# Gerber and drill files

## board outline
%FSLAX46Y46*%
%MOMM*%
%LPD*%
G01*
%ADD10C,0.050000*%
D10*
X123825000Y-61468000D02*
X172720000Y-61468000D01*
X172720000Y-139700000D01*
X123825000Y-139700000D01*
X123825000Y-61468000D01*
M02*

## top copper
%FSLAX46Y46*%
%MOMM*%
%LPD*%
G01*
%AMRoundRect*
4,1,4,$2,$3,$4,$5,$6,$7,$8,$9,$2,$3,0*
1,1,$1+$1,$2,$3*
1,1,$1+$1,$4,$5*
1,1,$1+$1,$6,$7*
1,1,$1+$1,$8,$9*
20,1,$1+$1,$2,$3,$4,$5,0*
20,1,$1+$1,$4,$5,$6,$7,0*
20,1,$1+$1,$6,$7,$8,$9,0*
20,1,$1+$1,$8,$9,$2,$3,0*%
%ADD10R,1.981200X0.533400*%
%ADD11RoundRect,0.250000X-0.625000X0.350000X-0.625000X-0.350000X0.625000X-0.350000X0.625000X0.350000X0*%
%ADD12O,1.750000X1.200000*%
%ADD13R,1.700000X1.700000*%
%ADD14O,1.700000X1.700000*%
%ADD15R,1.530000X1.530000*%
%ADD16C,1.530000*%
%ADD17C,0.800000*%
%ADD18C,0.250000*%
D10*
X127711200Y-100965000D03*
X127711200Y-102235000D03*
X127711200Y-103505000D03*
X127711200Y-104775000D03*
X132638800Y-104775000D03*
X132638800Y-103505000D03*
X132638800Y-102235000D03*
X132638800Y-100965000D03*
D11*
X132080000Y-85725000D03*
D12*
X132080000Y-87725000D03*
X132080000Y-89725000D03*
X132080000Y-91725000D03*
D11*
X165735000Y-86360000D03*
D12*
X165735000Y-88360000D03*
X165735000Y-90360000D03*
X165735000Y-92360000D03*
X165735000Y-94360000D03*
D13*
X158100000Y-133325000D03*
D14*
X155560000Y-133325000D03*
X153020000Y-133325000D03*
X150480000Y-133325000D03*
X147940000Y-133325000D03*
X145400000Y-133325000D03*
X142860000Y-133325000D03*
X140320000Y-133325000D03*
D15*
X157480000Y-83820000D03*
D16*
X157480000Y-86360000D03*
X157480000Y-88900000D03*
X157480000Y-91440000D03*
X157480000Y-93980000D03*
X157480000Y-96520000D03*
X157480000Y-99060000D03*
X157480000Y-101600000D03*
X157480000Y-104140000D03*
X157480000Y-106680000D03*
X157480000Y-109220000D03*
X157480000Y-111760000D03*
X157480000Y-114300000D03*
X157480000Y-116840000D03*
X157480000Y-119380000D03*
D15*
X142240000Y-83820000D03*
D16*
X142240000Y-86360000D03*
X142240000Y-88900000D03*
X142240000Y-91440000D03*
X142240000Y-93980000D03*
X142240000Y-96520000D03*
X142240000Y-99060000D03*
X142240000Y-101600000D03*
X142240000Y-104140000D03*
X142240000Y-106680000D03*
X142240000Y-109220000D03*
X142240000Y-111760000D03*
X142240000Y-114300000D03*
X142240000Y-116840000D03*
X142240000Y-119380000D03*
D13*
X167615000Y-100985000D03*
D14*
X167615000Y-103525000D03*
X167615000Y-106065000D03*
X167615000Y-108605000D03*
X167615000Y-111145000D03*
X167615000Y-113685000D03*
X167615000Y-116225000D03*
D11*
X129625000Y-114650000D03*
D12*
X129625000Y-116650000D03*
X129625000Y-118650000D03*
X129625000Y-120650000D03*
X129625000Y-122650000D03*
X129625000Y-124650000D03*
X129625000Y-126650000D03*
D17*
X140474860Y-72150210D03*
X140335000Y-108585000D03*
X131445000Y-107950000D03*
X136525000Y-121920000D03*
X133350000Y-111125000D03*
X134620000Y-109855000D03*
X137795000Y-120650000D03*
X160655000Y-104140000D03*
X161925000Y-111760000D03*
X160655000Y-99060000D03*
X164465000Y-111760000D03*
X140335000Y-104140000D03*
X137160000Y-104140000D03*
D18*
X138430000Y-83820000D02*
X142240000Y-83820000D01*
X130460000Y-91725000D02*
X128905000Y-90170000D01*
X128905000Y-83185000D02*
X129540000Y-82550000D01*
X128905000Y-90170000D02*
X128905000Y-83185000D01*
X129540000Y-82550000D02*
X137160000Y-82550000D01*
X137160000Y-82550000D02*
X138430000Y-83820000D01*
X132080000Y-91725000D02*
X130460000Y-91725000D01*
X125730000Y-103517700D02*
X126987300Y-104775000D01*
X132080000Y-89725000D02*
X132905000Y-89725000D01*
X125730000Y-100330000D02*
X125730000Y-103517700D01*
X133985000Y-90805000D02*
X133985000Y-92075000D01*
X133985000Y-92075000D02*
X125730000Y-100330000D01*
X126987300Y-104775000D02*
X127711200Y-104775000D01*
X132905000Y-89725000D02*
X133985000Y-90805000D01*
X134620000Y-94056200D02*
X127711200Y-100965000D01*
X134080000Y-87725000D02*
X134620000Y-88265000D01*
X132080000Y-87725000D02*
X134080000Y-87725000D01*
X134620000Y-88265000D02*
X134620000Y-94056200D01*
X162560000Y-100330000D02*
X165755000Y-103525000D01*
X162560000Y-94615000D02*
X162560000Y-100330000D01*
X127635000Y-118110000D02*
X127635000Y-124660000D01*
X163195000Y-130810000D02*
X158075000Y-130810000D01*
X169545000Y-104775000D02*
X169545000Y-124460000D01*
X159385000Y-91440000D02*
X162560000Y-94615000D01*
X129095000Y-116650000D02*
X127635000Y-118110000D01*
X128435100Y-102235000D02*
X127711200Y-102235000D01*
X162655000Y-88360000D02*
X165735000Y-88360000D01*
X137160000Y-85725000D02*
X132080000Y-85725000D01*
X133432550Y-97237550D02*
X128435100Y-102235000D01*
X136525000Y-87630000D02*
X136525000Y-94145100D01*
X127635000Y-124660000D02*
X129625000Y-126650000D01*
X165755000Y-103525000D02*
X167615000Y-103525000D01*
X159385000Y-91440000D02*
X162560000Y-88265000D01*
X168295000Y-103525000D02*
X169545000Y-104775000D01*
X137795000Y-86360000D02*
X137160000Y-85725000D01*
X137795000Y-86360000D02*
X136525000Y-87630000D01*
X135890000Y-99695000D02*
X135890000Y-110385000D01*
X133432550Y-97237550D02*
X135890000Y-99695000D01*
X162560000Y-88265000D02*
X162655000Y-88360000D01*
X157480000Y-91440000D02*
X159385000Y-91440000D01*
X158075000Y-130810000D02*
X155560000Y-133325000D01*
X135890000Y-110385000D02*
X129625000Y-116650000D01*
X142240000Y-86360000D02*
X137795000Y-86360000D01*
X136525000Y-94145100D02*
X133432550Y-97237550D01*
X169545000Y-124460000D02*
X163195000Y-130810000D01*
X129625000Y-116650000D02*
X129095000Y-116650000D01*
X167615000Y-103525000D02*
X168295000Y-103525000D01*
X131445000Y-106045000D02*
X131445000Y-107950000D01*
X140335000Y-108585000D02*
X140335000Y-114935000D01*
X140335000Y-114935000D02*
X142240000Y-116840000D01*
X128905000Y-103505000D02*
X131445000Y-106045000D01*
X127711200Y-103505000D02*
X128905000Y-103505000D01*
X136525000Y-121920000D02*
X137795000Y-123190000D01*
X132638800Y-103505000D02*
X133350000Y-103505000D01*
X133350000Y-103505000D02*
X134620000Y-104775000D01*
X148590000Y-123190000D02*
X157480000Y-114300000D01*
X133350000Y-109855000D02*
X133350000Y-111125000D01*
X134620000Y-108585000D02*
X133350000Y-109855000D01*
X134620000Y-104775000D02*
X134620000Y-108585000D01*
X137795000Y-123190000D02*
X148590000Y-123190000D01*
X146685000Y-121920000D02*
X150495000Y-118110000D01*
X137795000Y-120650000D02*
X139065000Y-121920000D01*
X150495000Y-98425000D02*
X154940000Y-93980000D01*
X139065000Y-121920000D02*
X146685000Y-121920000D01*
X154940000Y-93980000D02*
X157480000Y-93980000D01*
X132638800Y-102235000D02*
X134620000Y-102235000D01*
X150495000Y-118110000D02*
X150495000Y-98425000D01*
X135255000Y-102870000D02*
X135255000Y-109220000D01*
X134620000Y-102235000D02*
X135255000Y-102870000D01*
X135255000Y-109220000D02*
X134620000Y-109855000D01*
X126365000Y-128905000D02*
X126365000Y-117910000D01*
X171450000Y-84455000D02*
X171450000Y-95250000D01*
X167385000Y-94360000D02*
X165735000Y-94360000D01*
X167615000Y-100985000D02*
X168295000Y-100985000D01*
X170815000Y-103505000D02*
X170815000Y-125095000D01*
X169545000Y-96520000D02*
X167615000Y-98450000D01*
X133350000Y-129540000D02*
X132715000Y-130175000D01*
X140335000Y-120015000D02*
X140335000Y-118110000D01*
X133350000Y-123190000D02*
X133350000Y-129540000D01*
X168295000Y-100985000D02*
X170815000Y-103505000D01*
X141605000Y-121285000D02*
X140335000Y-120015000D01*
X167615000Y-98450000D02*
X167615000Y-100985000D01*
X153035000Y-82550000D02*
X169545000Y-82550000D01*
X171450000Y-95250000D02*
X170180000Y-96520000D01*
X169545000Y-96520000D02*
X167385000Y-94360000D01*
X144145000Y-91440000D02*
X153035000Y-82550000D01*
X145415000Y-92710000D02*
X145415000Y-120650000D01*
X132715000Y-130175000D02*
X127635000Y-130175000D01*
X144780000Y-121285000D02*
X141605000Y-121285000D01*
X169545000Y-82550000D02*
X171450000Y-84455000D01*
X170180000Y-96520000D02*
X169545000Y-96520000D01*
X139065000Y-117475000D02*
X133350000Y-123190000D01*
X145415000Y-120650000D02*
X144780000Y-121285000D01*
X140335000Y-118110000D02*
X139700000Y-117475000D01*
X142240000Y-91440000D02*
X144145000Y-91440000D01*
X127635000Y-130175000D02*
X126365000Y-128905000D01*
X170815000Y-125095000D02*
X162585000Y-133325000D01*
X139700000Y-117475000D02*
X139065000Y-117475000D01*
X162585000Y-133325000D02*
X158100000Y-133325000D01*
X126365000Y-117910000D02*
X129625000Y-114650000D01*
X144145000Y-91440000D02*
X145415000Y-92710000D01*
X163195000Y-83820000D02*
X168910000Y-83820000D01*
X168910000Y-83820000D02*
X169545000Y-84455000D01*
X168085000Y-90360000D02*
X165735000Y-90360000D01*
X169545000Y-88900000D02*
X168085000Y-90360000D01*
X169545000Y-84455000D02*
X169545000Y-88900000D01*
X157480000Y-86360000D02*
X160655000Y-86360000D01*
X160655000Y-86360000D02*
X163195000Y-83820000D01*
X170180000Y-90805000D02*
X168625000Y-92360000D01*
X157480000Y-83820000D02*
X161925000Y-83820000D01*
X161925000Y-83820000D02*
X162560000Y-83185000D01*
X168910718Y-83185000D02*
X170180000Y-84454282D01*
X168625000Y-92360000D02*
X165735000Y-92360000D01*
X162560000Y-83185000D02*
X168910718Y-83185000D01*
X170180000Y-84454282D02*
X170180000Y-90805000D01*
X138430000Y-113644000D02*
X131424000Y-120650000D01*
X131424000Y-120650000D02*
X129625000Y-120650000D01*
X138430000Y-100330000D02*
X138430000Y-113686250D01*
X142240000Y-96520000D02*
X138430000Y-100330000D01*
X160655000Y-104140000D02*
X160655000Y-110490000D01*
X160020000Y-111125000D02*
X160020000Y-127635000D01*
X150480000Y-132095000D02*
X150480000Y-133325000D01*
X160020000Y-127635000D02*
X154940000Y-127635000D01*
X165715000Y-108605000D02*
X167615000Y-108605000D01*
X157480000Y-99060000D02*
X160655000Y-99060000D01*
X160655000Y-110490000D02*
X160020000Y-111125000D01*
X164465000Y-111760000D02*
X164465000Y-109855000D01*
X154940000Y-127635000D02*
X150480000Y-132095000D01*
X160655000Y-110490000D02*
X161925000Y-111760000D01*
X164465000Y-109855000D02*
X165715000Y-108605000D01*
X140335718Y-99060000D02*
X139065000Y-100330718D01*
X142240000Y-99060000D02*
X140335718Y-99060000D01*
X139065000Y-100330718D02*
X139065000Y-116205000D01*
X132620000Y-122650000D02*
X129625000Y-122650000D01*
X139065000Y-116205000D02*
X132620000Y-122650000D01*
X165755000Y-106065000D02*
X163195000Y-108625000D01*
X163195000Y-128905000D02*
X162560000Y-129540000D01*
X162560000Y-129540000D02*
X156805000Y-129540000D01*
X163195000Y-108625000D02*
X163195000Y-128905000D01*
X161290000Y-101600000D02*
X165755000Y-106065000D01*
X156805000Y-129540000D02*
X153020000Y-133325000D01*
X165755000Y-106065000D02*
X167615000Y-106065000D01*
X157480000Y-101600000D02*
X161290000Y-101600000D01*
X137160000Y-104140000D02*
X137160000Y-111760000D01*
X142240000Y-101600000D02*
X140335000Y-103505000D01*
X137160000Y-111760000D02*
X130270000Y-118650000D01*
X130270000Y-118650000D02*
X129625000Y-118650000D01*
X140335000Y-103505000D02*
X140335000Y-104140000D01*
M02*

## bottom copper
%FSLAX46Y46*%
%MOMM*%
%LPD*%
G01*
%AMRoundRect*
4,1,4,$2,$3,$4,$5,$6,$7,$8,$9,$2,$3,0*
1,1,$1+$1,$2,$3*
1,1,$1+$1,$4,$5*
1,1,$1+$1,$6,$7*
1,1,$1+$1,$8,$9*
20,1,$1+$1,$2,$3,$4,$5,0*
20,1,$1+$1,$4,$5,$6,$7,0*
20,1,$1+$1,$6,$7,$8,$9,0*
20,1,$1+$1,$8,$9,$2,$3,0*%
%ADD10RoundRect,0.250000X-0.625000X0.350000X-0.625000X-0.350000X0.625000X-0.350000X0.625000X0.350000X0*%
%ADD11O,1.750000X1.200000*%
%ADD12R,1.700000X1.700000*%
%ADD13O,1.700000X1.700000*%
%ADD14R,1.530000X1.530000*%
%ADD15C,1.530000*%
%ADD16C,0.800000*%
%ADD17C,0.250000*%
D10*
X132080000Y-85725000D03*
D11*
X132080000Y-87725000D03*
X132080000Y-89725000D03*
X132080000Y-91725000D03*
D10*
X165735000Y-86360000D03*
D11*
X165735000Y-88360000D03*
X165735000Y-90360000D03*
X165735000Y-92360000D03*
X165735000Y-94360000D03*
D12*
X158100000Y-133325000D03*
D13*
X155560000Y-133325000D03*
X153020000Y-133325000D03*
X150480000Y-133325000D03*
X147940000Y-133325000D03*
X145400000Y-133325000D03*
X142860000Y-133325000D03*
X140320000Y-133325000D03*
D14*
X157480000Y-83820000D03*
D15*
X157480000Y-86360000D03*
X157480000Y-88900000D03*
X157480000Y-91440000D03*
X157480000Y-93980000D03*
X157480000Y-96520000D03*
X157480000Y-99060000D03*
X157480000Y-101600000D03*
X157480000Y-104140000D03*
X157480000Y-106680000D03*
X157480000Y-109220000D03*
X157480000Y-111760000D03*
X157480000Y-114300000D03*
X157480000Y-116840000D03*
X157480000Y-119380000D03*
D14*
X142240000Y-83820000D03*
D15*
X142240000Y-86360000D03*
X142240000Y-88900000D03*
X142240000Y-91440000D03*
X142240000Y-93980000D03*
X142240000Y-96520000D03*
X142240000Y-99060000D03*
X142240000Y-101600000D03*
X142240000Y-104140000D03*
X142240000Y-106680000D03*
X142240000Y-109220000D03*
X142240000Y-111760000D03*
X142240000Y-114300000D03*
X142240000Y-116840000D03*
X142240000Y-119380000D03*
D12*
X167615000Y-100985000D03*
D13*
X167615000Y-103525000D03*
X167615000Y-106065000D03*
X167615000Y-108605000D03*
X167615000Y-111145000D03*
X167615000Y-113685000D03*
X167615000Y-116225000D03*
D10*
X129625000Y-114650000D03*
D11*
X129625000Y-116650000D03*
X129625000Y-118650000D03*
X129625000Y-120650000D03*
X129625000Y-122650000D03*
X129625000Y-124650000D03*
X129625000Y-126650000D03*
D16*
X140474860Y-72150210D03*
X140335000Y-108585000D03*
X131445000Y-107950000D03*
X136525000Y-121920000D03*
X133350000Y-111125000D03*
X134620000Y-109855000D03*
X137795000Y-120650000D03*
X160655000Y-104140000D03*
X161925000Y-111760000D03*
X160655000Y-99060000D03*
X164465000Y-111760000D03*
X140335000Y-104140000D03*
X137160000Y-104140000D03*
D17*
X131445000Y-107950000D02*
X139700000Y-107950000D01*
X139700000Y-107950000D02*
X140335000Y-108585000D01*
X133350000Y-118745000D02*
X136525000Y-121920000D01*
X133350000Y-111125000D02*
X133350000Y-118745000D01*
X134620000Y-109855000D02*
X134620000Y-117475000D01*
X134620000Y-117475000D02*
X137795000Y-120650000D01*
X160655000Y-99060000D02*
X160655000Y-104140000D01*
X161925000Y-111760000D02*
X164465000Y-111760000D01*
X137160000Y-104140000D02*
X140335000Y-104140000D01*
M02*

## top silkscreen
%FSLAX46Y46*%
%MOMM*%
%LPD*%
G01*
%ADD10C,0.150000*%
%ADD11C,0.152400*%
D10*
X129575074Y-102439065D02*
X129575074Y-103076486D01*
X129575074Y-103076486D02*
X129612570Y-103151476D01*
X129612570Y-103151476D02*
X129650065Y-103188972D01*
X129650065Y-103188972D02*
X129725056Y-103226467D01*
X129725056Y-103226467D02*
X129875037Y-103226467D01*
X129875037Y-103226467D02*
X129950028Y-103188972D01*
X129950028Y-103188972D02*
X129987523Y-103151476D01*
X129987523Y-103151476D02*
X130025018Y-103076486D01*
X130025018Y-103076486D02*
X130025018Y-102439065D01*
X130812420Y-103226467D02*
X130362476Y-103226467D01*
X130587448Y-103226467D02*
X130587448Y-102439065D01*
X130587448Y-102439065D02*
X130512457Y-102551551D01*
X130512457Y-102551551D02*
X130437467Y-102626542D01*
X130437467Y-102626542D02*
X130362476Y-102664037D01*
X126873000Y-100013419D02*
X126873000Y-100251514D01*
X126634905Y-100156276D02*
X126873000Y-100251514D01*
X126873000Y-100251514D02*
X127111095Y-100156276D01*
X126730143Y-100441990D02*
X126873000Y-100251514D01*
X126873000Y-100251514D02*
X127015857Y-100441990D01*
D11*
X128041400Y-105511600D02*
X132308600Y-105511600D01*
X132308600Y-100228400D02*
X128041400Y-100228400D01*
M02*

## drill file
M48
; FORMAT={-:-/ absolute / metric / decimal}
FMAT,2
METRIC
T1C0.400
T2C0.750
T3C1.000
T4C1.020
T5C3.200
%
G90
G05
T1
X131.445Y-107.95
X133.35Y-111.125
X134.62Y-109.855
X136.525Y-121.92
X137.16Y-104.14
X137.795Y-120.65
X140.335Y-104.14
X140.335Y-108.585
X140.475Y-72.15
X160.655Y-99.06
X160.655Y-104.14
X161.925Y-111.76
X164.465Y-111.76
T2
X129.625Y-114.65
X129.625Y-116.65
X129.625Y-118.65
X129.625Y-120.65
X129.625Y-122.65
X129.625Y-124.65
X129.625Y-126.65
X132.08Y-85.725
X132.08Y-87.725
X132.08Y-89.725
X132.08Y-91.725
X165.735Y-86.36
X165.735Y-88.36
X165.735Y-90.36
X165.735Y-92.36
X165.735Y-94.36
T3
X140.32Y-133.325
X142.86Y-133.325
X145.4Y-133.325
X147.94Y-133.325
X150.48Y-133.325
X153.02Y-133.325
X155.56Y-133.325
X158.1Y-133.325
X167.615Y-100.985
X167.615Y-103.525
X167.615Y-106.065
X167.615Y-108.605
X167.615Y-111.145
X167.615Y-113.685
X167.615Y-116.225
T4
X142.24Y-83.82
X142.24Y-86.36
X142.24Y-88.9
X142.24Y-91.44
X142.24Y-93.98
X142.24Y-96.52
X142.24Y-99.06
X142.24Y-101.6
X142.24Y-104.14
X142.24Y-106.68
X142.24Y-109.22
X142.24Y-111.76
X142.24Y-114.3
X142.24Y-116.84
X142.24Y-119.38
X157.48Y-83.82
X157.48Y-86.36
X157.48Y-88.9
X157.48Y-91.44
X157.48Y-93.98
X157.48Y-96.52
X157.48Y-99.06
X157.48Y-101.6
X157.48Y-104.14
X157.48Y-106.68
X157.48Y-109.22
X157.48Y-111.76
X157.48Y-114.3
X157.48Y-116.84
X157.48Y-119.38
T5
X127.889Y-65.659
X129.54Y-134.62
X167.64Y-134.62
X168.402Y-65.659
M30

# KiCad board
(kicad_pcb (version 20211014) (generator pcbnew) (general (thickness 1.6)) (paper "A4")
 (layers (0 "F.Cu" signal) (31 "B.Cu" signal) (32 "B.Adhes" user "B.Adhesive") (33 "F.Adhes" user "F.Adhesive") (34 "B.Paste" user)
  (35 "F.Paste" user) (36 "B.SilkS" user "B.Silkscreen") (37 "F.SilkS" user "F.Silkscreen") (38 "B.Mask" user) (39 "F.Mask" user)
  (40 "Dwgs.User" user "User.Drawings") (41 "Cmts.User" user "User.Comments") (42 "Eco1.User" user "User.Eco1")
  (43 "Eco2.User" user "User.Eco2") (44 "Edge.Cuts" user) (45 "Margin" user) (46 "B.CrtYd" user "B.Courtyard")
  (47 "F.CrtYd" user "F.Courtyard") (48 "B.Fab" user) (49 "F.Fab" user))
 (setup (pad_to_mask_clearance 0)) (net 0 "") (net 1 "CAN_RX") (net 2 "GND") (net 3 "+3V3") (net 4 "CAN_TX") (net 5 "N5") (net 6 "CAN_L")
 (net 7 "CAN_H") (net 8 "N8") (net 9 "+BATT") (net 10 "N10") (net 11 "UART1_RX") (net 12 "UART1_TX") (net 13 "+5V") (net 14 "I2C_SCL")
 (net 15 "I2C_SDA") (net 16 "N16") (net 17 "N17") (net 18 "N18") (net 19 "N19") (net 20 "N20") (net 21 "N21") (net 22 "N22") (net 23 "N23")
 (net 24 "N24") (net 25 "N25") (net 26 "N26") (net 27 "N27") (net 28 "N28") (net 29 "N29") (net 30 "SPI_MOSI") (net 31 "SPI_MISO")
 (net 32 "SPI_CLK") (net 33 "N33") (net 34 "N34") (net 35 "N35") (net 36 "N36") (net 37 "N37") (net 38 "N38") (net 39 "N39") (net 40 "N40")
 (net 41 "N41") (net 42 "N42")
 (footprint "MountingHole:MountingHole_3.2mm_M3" (layer "F.Cu") (at 168.402 65.659)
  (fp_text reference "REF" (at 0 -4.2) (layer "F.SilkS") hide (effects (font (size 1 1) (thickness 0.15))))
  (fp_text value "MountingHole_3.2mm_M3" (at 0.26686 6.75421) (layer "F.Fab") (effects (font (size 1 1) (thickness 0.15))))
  (pad "" np_thru_hole circle locked (at 0 0) (size 3.2 3.2) (drill 3.2) (layers *.Cu *.Mask)))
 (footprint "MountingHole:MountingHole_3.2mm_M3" (layer "F.Cu") (at 129.54 134.62)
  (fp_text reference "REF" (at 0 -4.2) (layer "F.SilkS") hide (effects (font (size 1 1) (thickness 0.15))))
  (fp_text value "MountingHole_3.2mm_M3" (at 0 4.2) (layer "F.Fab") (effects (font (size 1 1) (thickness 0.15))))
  (pad "" np_thru_hole circle locked (at 0 0) (size 3.2 3.2) (drill 3.2) (layers *.Cu *.Mask)))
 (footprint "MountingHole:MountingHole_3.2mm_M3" (layer "F.Cu") (at 167.64 134.62)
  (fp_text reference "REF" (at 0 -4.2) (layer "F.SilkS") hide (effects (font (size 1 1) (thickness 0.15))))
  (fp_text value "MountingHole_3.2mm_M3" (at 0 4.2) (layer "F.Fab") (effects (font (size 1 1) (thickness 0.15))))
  (pad "" np_thru_hole circle locked (at 0 0) (size 3.2 3.2) (drill 3.2) (layers *.Cu *.Mask)))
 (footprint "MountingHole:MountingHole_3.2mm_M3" (layer "F.Cu") (at 127.889 65.659)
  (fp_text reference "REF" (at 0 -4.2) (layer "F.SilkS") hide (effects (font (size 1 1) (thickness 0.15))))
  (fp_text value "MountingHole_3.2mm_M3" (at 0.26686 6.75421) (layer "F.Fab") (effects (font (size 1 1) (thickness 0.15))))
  (pad "" np_thru_hole circle locked (at 0 0) (size 3.2 3.2) (drill 3.2) (layers *.Cu *.Mask)))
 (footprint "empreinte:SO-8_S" (layer "F.Cu") (at 130.175 102.87)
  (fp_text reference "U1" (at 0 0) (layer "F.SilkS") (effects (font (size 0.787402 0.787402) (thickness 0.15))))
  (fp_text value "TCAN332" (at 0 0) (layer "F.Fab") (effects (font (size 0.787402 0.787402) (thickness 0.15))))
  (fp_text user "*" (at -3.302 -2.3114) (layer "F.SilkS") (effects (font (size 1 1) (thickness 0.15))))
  (fp_line (start -2.1336 2.6416) (end 2.1336 2.6416) (layer "F.SilkS") (width 0.1524))
  (fp_line (start 2.1336 -2.6416) (end -2.1336 -2.6416) (layer "F.SilkS") (width 0.1524))
  (pad "1" smd rect locked (at -2.4638 -1.905) (size 1.9812 0.5334) (layers "F.Cu" "F.Paste" "F.Mask") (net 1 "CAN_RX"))
  (pad "2" smd rect locked (at -2.4638 -0.635) (size 1.9812 0.5334) (layers "F.Cu" "F.Paste" "F.Mask") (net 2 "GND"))
  (pad "3" smd rect locked (at -2.4638 0.635) (size 1.9812 0.5334) (layers "F.Cu" "F.Paste" "F.Mask") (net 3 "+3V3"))
  (pad "4" smd rect locked (at -2.4638 1.905) (size 1.9812 0.5334) (layers "F.Cu" "F.Paste" "F.Mask") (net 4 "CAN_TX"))
  (pad "5" smd rect locked (at 2.4638 1.905) (size 1.9812 0.5334) (layers "F.Cu" "F.Paste" "F.Mask") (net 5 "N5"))
  (pad "6" smd rect locked (at 2.4638 0.635) (size 1.9812 0.5334) (layers "F.Cu" "F.Paste" "F.Mask") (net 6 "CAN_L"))
  (pad "7" smd rect locked (at 2.4638 -0.635) (size 1.9812 0.5334) (layers "F.Cu" "F.Paste" "F.Mask") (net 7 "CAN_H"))
  (pad "8" smd rect locked (at 2.4638 -1.905) (size 1.9812 0.5334) (layers "F.Cu" "F.Paste" "F.Mask") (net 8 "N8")))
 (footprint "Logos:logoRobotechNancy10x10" (layer "B.Cu") (at 160.15986 70.37221 180)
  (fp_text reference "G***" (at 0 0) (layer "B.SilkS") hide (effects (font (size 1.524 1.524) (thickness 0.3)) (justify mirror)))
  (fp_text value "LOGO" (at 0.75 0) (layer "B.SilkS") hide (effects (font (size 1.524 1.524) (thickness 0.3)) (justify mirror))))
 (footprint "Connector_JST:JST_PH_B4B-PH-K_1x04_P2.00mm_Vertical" (layer "B.Cu") (at 132.08 85.725 -90)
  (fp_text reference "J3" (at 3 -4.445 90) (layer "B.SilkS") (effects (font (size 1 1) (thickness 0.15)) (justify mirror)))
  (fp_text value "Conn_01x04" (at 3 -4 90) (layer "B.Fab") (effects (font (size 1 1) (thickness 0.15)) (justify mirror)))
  (pad "1" thru_hole roundrect locked (at 0 0 270) (size 1.2 1.75) (drill 0.75) (layers *.Cu *.Mask) (roundrect_rratio 0.208333)
   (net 2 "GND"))
  (pad "2" thru_hole oval locked (at 2 0 270) (size 1.2 1.75) (drill 0.75) (layers *.Cu *.Mask) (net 1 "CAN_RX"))
  (pad "3" thru_hole oval locked (at 4 0 270) (size 1.2 1.75) (drill 0.75) (layers *.Cu *.Mask) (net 4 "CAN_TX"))
  (pad "4" thru_hole oval locked (at 6 0 270) (size 1.2 1.75) (drill 0.75) (layers *.Cu *.Mask) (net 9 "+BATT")))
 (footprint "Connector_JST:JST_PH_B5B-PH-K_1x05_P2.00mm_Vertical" (layer "B.Cu") (at 165.735 86.36 -90)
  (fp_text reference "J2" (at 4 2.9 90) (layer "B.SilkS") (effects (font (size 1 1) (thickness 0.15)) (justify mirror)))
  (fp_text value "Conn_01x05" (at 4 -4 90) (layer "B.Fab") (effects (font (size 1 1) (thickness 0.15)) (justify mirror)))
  (pad "1" thru_hole roundrect locked (at 0 0 270) (size 1.2 1.75) (drill 0.75) (layers *.Cu *.Mask) (roundrect_rratio 0.208333)
   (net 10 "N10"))
  (pad "2" thru_hole oval locked (at 2 0 270) (size 1.2 1.75) (drill 0.75) (layers *.Cu *.Mask) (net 2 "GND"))
  (pad "3" thru_hole oval locked (at 4 0 270) (size 1.2 1.75) (drill 0.75) (layers *.Cu *.Mask) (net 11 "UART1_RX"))
  (pad "4" thru_hole oval locked (at 6 0 270) (size 1.2 1.75) (drill 0.75) (layers *.Cu *.Mask) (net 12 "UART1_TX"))
  (pad "5" thru_hole oval locked (at 8 0 270) (size 1.2 1.75) (drill 0.75) (layers *.Cu *.Mask) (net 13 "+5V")))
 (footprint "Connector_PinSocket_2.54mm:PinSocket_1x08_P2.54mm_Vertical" (layer "B.Cu") (at 158.1 133.325 90)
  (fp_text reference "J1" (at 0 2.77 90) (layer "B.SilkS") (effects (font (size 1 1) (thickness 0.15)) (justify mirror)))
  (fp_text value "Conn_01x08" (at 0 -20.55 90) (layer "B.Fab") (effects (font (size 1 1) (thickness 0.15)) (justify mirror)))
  (pad "1" thru_hole rect locked (at 0 0 90) (size 1.7 1.7) (drill 1) (layers *.Cu *.Mask) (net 13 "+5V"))
  (pad "2" thru_hole oval locked (at 0 -2.54 90) (size 1.7 1.7) (drill 1) (layers *.Cu *.Mask) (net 2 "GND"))
  (pad "3" thru_hole oval locked (at 0 -5.08 90) (size 1.7 1.7) (drill 1) (layers *.Cu *.Mask) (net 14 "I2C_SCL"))
  (pad "4" thru_hole oval locked (at 0 -7.62 90) (size 1.7 1.7) (drill 1) (layers *.Cu *.Mask) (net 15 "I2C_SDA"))
  (pad "5" thru_hole oval locked (at 0 -10.16 90) (size 1.7 1.7) (drill 1) (layers *.Cu *.Mask) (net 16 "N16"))
  (pad "6" thru_hole oval locked (at 0 -12.7 90) (size 1.7 1.7) (drill 1) (layers *.Cu *.Mask) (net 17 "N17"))
  (pad "7" thru_hole oval locked (at 0 -15.24 90) (size 1.7 1.7) (drill 1) (layers *.Cu *.Mask) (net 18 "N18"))
  (pad "8" thru_hole oval locked (at 0 -17.78 90) (size 1.7 1.7) (drill 1) (layers *.Cu *.Mask) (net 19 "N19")))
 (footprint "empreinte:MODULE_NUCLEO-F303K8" (layer "B.Cu") (at 149.86 101.6 180)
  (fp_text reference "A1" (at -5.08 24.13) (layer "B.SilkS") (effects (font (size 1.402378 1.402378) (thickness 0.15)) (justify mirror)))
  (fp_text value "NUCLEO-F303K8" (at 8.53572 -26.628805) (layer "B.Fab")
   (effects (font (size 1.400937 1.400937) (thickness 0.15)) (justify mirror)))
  (pad "3.1" thru_hole rect locked (at -7.62 17.78 180) (size 1.53 1.53) (drill 1.02) (layers *.Cu *.Mask) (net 12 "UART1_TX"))
  (pad "3.2" thru_hole circle locked (at -7.62 15.24 180) (size 1.53 1.53) (drill 1.02) (layers *.Cu *.Mask) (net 11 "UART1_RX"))
  (pad "3.3" thru_hole circle locked (at -7.62 12.7 180) (size 1.53 1.53) (drill 1.02) (layers *.Cu *.Mask) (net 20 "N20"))
  (pad "3.4" thru_hole circle locked (at -7.62 10.16 180) (size 1.53 1.53) (drill 1.02) (layers *.Cu *.Mask) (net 2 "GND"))
  (pad "3.5" thru_hole circle locked (at -7.62 7.62 180) (size 1.53 1.53) (drill 1.02) (layers *.Cu *.Mask) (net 7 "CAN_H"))
  (pad "3.6" thru_hole circle locked (at -7.62 5.08 180) (size 1.53 1.53) (drill 1.02) (layers *.Cu *.Mask) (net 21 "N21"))
  (pad "3.7" thru_hole circle locked (at -7.62 2.54 180) (size 1.53 1.53) (drill 1.02) (layers *.Cu *.Mask) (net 15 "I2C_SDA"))
  (pad "3.8" thru_hole circle locked (at -7.62 0 180) (size 1.53 1.53) (drill 1.02) (layers *.Cu *.Mask) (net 14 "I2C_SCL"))
  (pad "3.9" thru_hole circle locked (at -7.62 -2.54 180) (size 1.53 1.53) (drill 1.02) (layers *.Cu *.Mask) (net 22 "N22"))
  (pad "3.10" thru_hole circle locked (at -7.62 -5.08 180) (size 1.53 1.53) (drill 1.02) (layers *.Cu *.Mask) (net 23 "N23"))
  (pad "3.11" thru_hole circle locked (at -7.62 -7.62 180) (size 1.53 1.53) (drill 1.02) (layers *.Cu *.Mask) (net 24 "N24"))
  (pad "3.12" thru_hole circle locked (at -7.62 -10.16 180) (size 1.53 1.53) (drill 1.02) (layers *.Cu *.Mask) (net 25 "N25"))
  (pad "3.13" thru_hole circle locked (at -7.62 -12.7 180) (size 1.53 1.53) (drill 1.02) (layers *.Cu *.Mask) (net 6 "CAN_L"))
  (pad "3.14" thru_hole circle locked (at -7.62 -15.24 180) (size 1.53 1.53) (drill 1.02) (layers *.Cu *.Mask) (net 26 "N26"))
  (pad "3.15" thru_hole circle locked (at -7.62 -17.78 180) (size 1.53 1.53) (drill 1.02) (layers *.Cu *.Mask) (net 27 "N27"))
  (pad "4.1" thru_hole rect locked (at 7.62 17.78 180) (size 1.53 1.53) (drill 1.02) (layers *.Cu *.Mask) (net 9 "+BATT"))
  (pad "4.2" thru_hole circle locked (at 7.62 15.24 180) (size 1.53 1.53) (drill 1.02) (layers *.Cu *.Mask) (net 2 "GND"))
  (pad "4.3" thru_hole circle locked (at 7.62 12.7 180) (size 1.53 1.53) (drill 1.02) (layers *.Cu *.Mask) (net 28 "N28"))
  (pad "4.4" thru_hole circle locked (at 7.62 10.16 180) (size 1.53 1.53) (drill 1.02) (layers *.Cu *.Mask) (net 13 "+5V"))
  (pad "4.5" thru_hole circle locked (at 7.62 7.62 180) (size 1.53 1.53) (drill 1.02) (layers *.Cu *.Mask) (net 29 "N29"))
  (pad "4.6" thru_hole circle locked (at 7.62 5.08 180) (size 1.53 1.53) (drill 1.02) (layers *.Cu *.Mask) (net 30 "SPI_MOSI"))
  (pad "4.7" thru_hole circle locked (at 7.62 2.54 180) (size 1.53 1.53) (drill 1.02) (layers *.Cu *.Mask) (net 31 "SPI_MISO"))
  (pad "4.8" thru_hole circle locked (at 7.62 0 180) (size 1.53 1.53) (drill 1.02) (layers *.Cu *.Mask) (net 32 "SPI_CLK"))
  (pad "4.9" thru_hole circle locked (at 7.62 -2.54 180) (size 1.53 1.53) (drill 1.02) (layers *.Cu *.Mask) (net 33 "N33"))
  (pad "4.10" thru_hole circle locked (at 7.62 -5.08 180) (size 1.53 1.53) (drill 1.02) (layers *.Cu *.Mask) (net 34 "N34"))
  (pad "4.11" thru_hole circle locked (at 7.62 -7.62 180) (size 1.53 1.53) (drill 1.02) (layers *.Cu *.Mask) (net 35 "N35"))
  (pad "4.12" thru_hole circle locked (at 7.62 -10.16 180) (size 1.53 1.53) (drill 1.02) (layers *.Cu *.Mask) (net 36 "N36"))
  (pad "4.13" thru_hole circle locked (at 7.62 -12.7 180) (size 1.53 1.53) (drill 1.02) (layers *.Cu *.Mask) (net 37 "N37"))
  (pad "4.14" thru_hole circle locked (at 7.62 -15.24 180) (size 1.53 1.53) (drill 1.02) (layers *.Cu *.Mask) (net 3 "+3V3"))
  (pad "4.15" thru_hole circle locked (at 7.62 -17.78 180) (size 1.53 1.53) (drill 1.02) (layers *.Cu *.Mask) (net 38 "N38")))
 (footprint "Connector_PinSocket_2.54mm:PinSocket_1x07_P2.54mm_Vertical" (layer "B.Cu") (at 167.615 100.985 180)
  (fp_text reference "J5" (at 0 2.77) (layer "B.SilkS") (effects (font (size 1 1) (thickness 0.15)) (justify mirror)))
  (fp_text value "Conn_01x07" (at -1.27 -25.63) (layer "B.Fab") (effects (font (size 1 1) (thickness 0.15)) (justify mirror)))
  (pad "1" thru_hole rect locked (at 0 0 180) (size 1.7 1.7) (drill 1) (layers *.Cu *.Mask) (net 13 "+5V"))
  (pad "2" thru_hole oval locked (at 0 -2.54 180) (size 1.7 1.7) (drill 1) (layers *.Cu *.Mask) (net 2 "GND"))
  (pad "3" thru_hole oval locked (at 0 -5.08 180) (size 1.7 1.7) (drill 1) (layers *.Cu *.Mask) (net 14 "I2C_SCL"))
  (pad "4" thru_hole oval locked (at 0 -7.62 180) (size 1.7 1.7) (drill 1) (layers *.Cu *.Mask) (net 15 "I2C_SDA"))
  (pad "5" thru_hole oval locked (at 0 -10.16 180) (size 1.7 1.7) (drill 1) (layers *.Cu *.Mask) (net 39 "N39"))
  (pad "6" thru_hole oval locked (at 0 -12.7 180) (size 1.7 1.7) (drill 1) (layers *.Cu *.Mask) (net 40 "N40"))
  (pad "7" thru_hole oval locked (at 0 -15.24 180) (size 1.7 1.7) (drill 1) (layers *.Cu *.Mask) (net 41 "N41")))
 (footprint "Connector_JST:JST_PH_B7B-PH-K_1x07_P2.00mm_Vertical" (layer "B.Cu") (at 129.625 114.65 -90)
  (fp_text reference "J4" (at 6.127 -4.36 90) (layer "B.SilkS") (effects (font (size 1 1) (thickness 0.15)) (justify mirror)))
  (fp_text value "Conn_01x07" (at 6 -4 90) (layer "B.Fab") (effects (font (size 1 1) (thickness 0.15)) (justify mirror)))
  (pad "1" thru_hole roundrect locked (at 0 0 270) (size 1.2 1.75) (drill 0.75) (layers *.Cu *.Mask) (roundrect_rratio 0.208333)
   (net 13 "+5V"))
  (pad "2" thru_hole oval locked (at 2 0 270) (size 1.2 1.75) (drill 0.75) (layers *.Cu *.Mask) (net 2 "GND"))
  (pad "3" thru_hole oval locked (at 4 0 270) (size 1.2 1.75) (drill 0.75) (layers *.Cu *.Mask) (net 32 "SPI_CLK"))
  (pad "4" thru_hole oval locked (at 6 0 270) (size 1.2 1.75) (drill 0.75) (layers *.Cu *.Mask) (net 30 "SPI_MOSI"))
  (pad "5" thru_hole oval locked (at 8 0 270) (size 1.2 1.75) (drill 0.75) (layers *.Cu *.Mask) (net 31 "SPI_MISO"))
  (pad "6" thru_hole oval locked (at 10 0 270) (size 1.2 1.75) (drill 0.75) (layers *.Cu *.Mask) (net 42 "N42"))
  (pad "7" thru_hole oval locked (at 12 0 270) (size 1.2 1.75) (drill 0.75) (layers *.Cu *.Mask) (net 2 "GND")))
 (gr_rect (start 123.825 61.468) (end 172.72 139.7) (layer "Edge.Cuts") (width 0.05) (fill none))
 (via (at 140.47486 72.15021) (size 0.8) (drill 0.4) (layers "F.Cu" "B.Cu") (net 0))
 (segment (start 138.43 83.82) (end 142.24 83.82) (width 0.25) (layer "F.Cu") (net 9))
 (segment (start 130.46 91.725) (end 128.905 90.17) (width 0.25) (layer "F.Cu") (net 9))
 (segment (start 128.905 83.185) (end 129.54 82.55) (width 0.25) (layer "F.Cu") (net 9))
 (segment (start 128.905 90.17) (end 128.905 83.185) (width 0.25) (layer "F.Cu") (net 9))
 (segment (start 129.54 82.55) (end 137.16 82.55) (width 0.25) (layer "F.Cu") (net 9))
 (segment (start 137.16 82.55) (end 138.43 83.82) (width 0.25) (layer "F.Cu") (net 9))
 (segment (start 132.08 91.725) (end 130.46 91.725) (width 0.25) (layer "F.Cu") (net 9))
 (segment (start 125.73 103.5177) (end 126.9873 104.775) (width 0.25) (layer "F.Cu") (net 4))
 (segment (start 132.08 89.725) (end 132.905 89.725) (width 0.25) (layer "F.Cu") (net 4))
 (segment (start 125.73 100.33) (end 125.73 103.5177) (width 0.25) (layer "F.Cu") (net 4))
 (segment (start 133.985 90.805) (end 133.985 92.075) (width 0.25) (layer "F.Cu") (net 4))
 (segment (start 133.985 92.075) (end 125.73 100.33) (width 0.25) (layer "F.Cu") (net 4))
 (segment (start 126.9873 104.775) (end 127.7112 104.775) (width 0.25) (layer "F.Cu") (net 4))
 (segment (start 132.905 89.725) (end 133.985 90.805) (width 0.25) (layer "F.Cu") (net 4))
 (segment (start 134.62 94.0562) (end 127.7112 100.965) (width 0.25) (layer "F.Cu") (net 1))
 (segment (start 134.08 87.725) (end 134.62 88.265) (width 0.25) (layer "F.Cu") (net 1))
 (segment (start 132.08 87.725) (end 134.08 87.725) (width 0.25) (layer "F.Cu") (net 1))
 (segment (start 134.62 88.265) (end 134.62 94.0562) (width 0.25) (layer "F.Cu") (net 1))
 (segment (start 162.56 100.33) (end 165.755 103.525) (width 0.25) (layer "F.Cu") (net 2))
 (segment (start 162.56 94.615) (end 162.56 100.33) (width 0.25) (layer "F.Cu") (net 2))
 (segment (start 127.635 118.11) (end 127.635 124.66) (width 0.25) (layer "F.Cu") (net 2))
 (segment (start 163.195 130.81) (end 158.075 130.81) (width 0.25) (layer "F.Cu") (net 2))
 (segment (start 169.545 104.775) (end 169.545 124.46) (width 0.25) (layer "F.Cu") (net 2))
 (segment (start 159.385 91.44) (end 162.56 94.615) (width 0.25) (layer "F.Cu") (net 2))
 (segment (start 129.095 116.65) (end 127.635 118.11) (width 0.25) (layer "F.Cu") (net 2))
 (segment (start 128.4351 102.235) (end 127.7112 102.235) (width 0.25) (layer "F.Cu") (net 2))
 (segment (start 162.655 88.36) (end 165.735 88.36) (width 0.25) (layer "F.Cu") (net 2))
 (segment (start 137.16 85.725) (end 132.08 85.725) (width 0.25) (layer "F.Cu") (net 2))
 (segment (start 133.43255 97.23755) (end 128.4351 102.235) (width 0.25) (layer "F.Cu") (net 2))
 (segment (start 136.525 87.63) (end 136.525 94.1451) (width 0.25) (layer "F.Cu") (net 2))
 (segment (start 127.635 124.66) (end 129.625 126.65) (width 0.25) (layer "F.Cu") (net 2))
 (segment (start 165.755 103.525) (end 167.615 103.525) (width 0.25) (layer "F.Cu") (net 2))
 (segment (start 159.385 91.44) (end 162.56 88.265) (width 0.25) (layer "F.Cu") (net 2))
 (segment (start 168.295 103.525) (end 169.545 104.775) (width 0.25) (layer "F.Cu") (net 2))
 (segment (start 137.795 86.36) (end 137.16 85.725) (width 0.25) (layer "F.Cu") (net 2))
 (segment (start 137.795 86.36) (end 136.525 87.63) (width 0.25) (layer "F.Cu") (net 2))
 (segment (start 135.89 99.695) (end 135.89 110.385) (width 0.25) (layer "F.Cu") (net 2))
 (segment (start 133.43255 97.23755) (end 135.89 99.695) (width 0.25) (layer "F.Cu") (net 2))
 (segment (start 162.56 88.265) (end 162.655 88.36) (width 0.25) (layer "F.Cu") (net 2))
 (segment (start 157.48 91.44) (end 159.385 91.44) (width 0.25) (layer "F.Cu") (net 2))
 (segment (start 158.075 130.81) (end 155.56 133.325) (width 0.25) (layer "F.Cu") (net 2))
 (segment (start 135.89 110.385) (end 129.625 116.65) (width 0.25) (layer "F.Cu") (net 2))
 (segment (start 142.24 86.36) (end 137.795 86.36) (width 0.25) (layer "F.Cu") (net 2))
 (segment (start 136.525 94.1451) (end 133.43255 97.23755) (width 0.25) (layer "F.Cu") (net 2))
 (segment (start 169.545 124.46) (end 163.195 130.81) (width 0.25) (layer "F.Cu") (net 2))
 (segment (start 129.625 116.65) (end 129.095 116.65) (width 0.25) (layer "F.Cu") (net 2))
 (segment (start 167.615 103.525) (end 168.295 103.525) (width 0.25) (layer "F.Cu") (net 2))
 (segment (start 131.445 106.045) (end 131.445 107.95) (width 0.25) (layer "F.Cu") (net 3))
 (segment (start 140.335 108.585) (end 140.335 114.935) (width 0.25) (layer "F.Cu") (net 3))
 (segment (start 140.335 114.935) (end 142.24 116.84) (width 0.25) (layer "F.Cu") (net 3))
 (segment (start 128.905 103.505) (end 131.445 106.045) (width 0.25) (layer "F.Cu") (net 3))
 (segment (start 127.7112 103.505) (end 128.905 103.505) (width 0.25) (layer "F.Cu") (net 3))
 (via (at 140.335 108.585) (size 0.8) (drill 0.4) (layers "F.Cu" "B.Cu") (free) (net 3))
 (via (at 131.445 107.95) (size 0.8) (drill 0.4) (layers "F.Cu" "B.Cu") (free) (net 3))
 (segment (start 131.445 107.95) (end 139.7 107.95) (width 0.25) (layer "B.Cu") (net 3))
 (segment (start 139.7 107.95) (end 140.335 108.585) (width 0.25) (layer "B.Cu") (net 3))
 (segment (start 136.525 121.92) (end 137.795 123.19) (width 0.25) (layer "F.Cu") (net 6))
 (segment (start 132.6388 103.505) (end 133.35 103.505) (width 0.25) (layer "F.Cu") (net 6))
 (segment (start 133.35 103.505) (end 134.62 104.775) (width 0.25) (layer "F.Cu") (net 6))
 (segment (start 148.59 123.19) (end 157.48 114.3) (width 0.25) (layer "F.Cu") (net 6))
 (segment (start 133.35 109.855) (end 133.35 111.125) (width 0.25) (layer "F.Cu") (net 6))
 (segment (start 134.62 108.585) (end 133.35 109.855) (width 0.25) (layer "F.Cu") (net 6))
 (segment (start 134.62 104.775) (end 134.62 108.585) (width 0.25) (layer "F.Cu") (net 6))
 (segment (start 137.795 123.19) (end 148.59 123.19) (width 0.25) (layer "F.Cu") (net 6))
 (via (at 136.525 121.92) (size 0.8) (drill 0.4) (layers "F.Cu" "B.Cu") (free) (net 6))
 (via (at 133.35 111.125) (size 0.8) (drill 0.4) (layers "F.Cu" "B.Cu") (free) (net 6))
 (segment (start 133.35 118.745) (end 136.525 121.92) (width 0.25) (layer "B.Cu") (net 6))
 (segment (start 133.35 111.125) (end 133.35 118.745) (width 0.25) (layer "B.Cu") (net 6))
 (segment (start 146.685 121.92) (end 150.495 118.11) (width 0.25) (layer "F.Cu") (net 7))
 (segment (start 137.795 120.65) (end 139.065 121.92) (width 0.25) (layer "F.Cu") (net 7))
 (segment (start 150.495 98.425) (end 154.94 93.98) (width 0.25) (layer "F.Cu") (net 7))
 (segment (start 139.065 121.92) (end 146.685 121.92) (width 0.25) (layer "F.Cu") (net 7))
 (segment (start 154.94 93.98) (end 157.48 93.98) (width 0.25) (layer "F.Cu") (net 7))
 (segment (start 132.6388 102.235) (end 134.62 102.235) (width 0.25) (layer "F.Cu") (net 7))
 (segment (start 150.495 118.11) (end 150.495 98.425) (width 0.25) (layer "F.Cu") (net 7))
 (segment (start 135.255 102.87) (end 135.255 109.22) (width 0.25) (layer "F.Cu") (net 7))
 (segment (start 134.62 102.235) (end 135.255 102.87) (width 0.25) (layer "F.Cu") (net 7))
 (segment (start 135.255 109.22) (end 134.62 109.855) (width 0.25) (layer "F.Cu") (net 7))
 (via (at 134.62 109.855) (size 0.8) (drill 0.4) (layers "F.Cu" "B.Cu") (free) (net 7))
 (via (at 137.795 120.65) (size 0.8) (drill 0.4) (layers "F.Cu" "B.Cu") (free) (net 7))
 (segment (start 134.62 109.855) (end 134.62 117.475) (width 0.25) (layer "B.Cu") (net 7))
 (segment (start 134.62 117.475) (end 137.795 120.65) (width 0.25) (layer "B.Cu") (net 7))
 (segment (start 126.365 128.905) (end 126.365 117.91) (width 0.25) (layer "F.Cu") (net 13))
 (segment (start 171.45 84.455) (end 171.45 95.25) (width 0.25) (layer "F.Cu") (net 13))
 (segment (start 167.385 94.36) (end 165.735 94.36) (width 0.25) (layer "F.Cu") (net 13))
 (segment (start 167.615 100.985) (end 168.295 100.985) (width 0.25) (layer "F.Cu") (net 13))
 (segment (start 170.815 103.505) (end 170.815 125.095) (width 0.25) (layer "F.Cu") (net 13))
 (segment (start 169.545 96.52) (end 167.615 98.45) (width 0.25) (layer "F.Cu") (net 13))
 (segment (start 133.35 129.54) (end 132.715 130.175) (width 0.25) (layer "F.Cu") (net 13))
 (segment (start 140.335 120.015) (end 140.335 118.11) (width 0.25) (layer "F.Cu") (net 13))
 (segment (start 133.35 123.19) (end 133.35 129.54) (width 0.25) (layer "F.Cu") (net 13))
 (segment (start 168.295 100.985) (end 170.815 103.505) (width 0.25) (layer "F.Cu") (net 13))
 (segment (start 141.605 121.285) (end 140.335 120.015) (width 0.25) (layer "F.Cu") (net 13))
 (segment (start 167.615 98.45) (end 167.615 100.985) (width 0.25) (layer "F.Cu") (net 13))
 (segment (start 153.035 82.55) (end 169.545 82.55) (width 0.25) (layer "F.Cu") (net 13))
 (segment (start 171.45 95.25) (end 170.18 96.52) (width 0.25) (layer "F.Cu") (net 13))
 (segment (start 169.545 96.52) (end 167.385 94.36) (width 0.25) (layer "F.Cu") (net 13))
 (segment (start 144.145 91.44) (end 153.035 82.55) (width 0.25) (layer "F.Cu") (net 13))
 (segment (start 145.415 92.71) (end 145.415 120.65) (width 0.25) (layer "F.Cu") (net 13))
 (segment (start 132.715 130.175) (end 127.635 130.175) (width 0.25) (layer "F.Cu") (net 13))
 (segment (start 144.78 121.285) (end 141.605 121.285) (width 0.25) (layer "F.Cu") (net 13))
 (segment (start 169.545 82.55) (end 171.45 84.455) (width 0.25) (layer "F.Cu") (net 13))
 (segment (start 170.18 96.52) (end 169.545 96.52) (width 0.25) (layer "F.Cu") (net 13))
 (segment (start 139.065 117.475) (end 133.35 123.19) (width 0.25) (layer "F.Cu") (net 13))
 (segment (start 145.415 120.65) (end 144.78 121.285) (width 0.25) (layer "F.Cu") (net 13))
 (segment (start 140.335 118.11) (end 139.7 117.475) (width 0.25) (layer "F.Cu") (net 13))
 (segment (start 142.24 91.44) (end 144.145 91.44) (width 0.25) (layer "F.Cu") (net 13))
 (segment (start 127.635 130.175) (end 126.365 128.905) (width 0.25) (layer "F.Cu") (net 13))
 (segment (start 170.815 125.095) (end 162.585 133.325) (width 0.25) (layer "F.Cu") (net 13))
 (segment (start 139.7 117.475) (end 139.065 117.475) (width 0.25) (layer "F.Cu") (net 13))
 (segment (start 162.585 133.325) (end 158.1 133.325) (width 0.25) (layer "F.Cu") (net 13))
 (segment (start 126.365 117.91) (end 129.625 114.65) (width 0.25) (layer "F.Cu") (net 13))
 (segment (start 144.145 91.44) (end 145.415 92.71) (width 0.25) (layer "F.Cu") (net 13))
 (segment (start 163.195 83.82) (end 168.91 83.82) (width 0.25) (layer "F.Cu") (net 11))
 (segment (start 168.91 83.82) (end 169.545 84.455) (width 0.25) (layer "F.Cu") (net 11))
 (segment (start 168.085 90.36) (end 165.735 90.36) (width 0.25) (layer "F.Cu") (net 11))
 (segment (start 169.545 88.9) (end 168.085 90.36) (width 0.25) (layer "F.Cu") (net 11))
 (segment (start 169.545 84.455) (end 169.545 88.9) (width 0.25) (layer "F.Cu") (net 11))
 (segment (start 157.48 86.36) (end 160.655 86.36) (width 0.25) (layer "F.Cu") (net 11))
 (segment (start 160.655 86.36) (end 163.195 83.82) (width 0.25) (layer "F.Cu") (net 11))
 (segment (start 170.18 90.805) (end 168.625 92.36) (width 0.25) (layer "F.Cu") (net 12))
 (segment (start 157.48 83.82) (end 161.925 83.82) (width 0.25) (layer "F.Cu") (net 12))
 (segment (start 161.925 83.82) (end 162.56 83.185) (width 0.25) (layer "F.Cu") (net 12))
 (segment (start 168.910718 83.185) (end 170.18 84.454282) (width 0.25) (layer "F.Cu") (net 12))
 (segment (start 168.625 92.36) (end 165.735 92.36) (width 0.25) (layer "F.Cu") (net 12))
 (segment (start 162.56 83.185) (end 168.910718 83.185) (width 0.25) (layer "F.Cu") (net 12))
 (segment (start 170.18 84.454282) (end 170.18 90.805) (width 0.25) (layer "F.Cu") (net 12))
 (segment (start 138.43 113.644) (end 131.424 120.65) (width 0.25) (layer "F.Cu") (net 30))
 (segment (start 131.424 120.65) (end 129.625 120.65) (width 0.25) (layer "F.Cu") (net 30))
 (segment (start 138.43 100.33) (end 138.43 113.68625) (width 0.25) (layer "F.Cu") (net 30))
 (segment (start 142.24 96.52) (end 138.43 100.33) (width 0.25) (layer "F.Cu") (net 30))
 (segment (start 160.655 104.14) (end 160.655 110.49) (width 0.25) (layer "F.Cu") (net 15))
 (segment (start 160.02 111.125) (end 160.02 127.635) (width 0.25) (layer "F.Cu") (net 15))
 (segment (start 150.48 132.095) (end 150.48 133.325) (width 0.25) (layer "F.Cu") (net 15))
 (segment (start 160.02 127.635) (end 154.94 127.635) (width 0.25) (layer "F.Cu") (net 15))
 (segment (start 165.715 108.605) (end 167.615 108.605) (width 0.25) (layer "F.Cu") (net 15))
 (segment (start 157.48 99.06) (end 160.655 99.06) (width 0.25) (layer "F.Cu") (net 15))
 (segment (start 160.655 110.49) (end 160.02 111.125) (width 0.25) (layer "F.Cu") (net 15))
 (segment (start 164.465 111.76) (end 164.465 109.855) (width 0.25) (layer "F.Cu") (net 15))
 (segment (start 154.94 127.635) (end 150.48 132.095) (width 0.25) (layer "F.Cu") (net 15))
 (segment (start 160.655 110.49) (end 161.925 111.76) (width 0.25) (layer "F.Cu") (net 15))
 (segment (start 164.465 109.855) (end 165.715 108.605) (width 0.25) (layer "F.Cu") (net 15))
 (via (at 160.655 104.14) (size 0.8) (drill 0.4) (layers "F.Cu" "B.Cu") (free) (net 15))
 (via (at 161.925 111.76) (size 0.8) (drill 0.4) (layers "F.Cu" "B.Cu") (free) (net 15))
 (via (at 160.655 99.06) (size 0.8) (drill 0.4) (layers "F.Cu" "B.Cu") (free) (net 15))
 (via (at 164.465 111.76) (size 0.8) (drill 0.4) (layers "F.Cu" "B.Cu") (free) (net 15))
 (segment (start 160.655 99.06) (end 160.655 104.14) (width 0.25) (layer "B.Cu") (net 15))
 (segment (start 161.925 111.76) (end 164.465 111.76) (width 0.25) (layer "B.Cu") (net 15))
 (segment (start 140.335718 99.06) (end 139.065 100.330718) (width 0.25) (layer "F.Cu") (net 31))
 (segment (start 142.24 99.06) (end 140.335718 99.06) (width 0.25) (layer "F.Cu") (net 31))
 (segment (start 139.065 100.330718) (end 139.065 116.205) (width 0.25) (layer "F.Cu") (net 31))
 (segment (start 132.62 122.65) (end 129.625 122.65) (width 0.25) (layer "F.Cu") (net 31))
 (segment (start 139.065 116.205) (end 132.62 122.65) (width 0.25) (layer "F.Cu") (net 31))
 (segment (start 165.755 106.065) (end 163.195 108.625) (width 0.25) (layer "F.Cu") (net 14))
 (segment (start 163.195 128.905) (end 162.56 129.54) (width 0.25) (layer "F.Cu") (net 14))
 (segment (start 162.56 129.54) (end 156.805 129.54) (width 0.25) (layer "F.Cu") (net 14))
 (segment (start 163.195 108.625) (end 163.195 128.905) (width 0.25) (layer "F.Cu") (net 14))
 (segment (start 161.29 101.6) (end 165.755 106.065) (width 0.25) (layer "F.Cu") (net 14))
 (segment (start 156.805 129.54) (end 153.02 133.325) (width 0.25) (layer "F.Cu") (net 14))
 (segment (start 165.755 106.065) (end 167.615 106.065) (width 0.25) (layer "F.Cu") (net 14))
 (segment (start 157.48 101.6) (end 161.29 101.6) (width 0.25) (layer "F.Cu") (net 14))
 (segment (start 137.16 104.14) (end 137.16 111.76) (width 0.25) (layer "F.Cu") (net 32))
 (segment (start 142.24 101.6) (end 140.335 103.505) (width 0.25) (layer "F.Cu") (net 32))
 (segment (start 137.16 111.76) (end 130.27 118.65) (width 0.25) (layer "F.Cu") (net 32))
 (segment (start 130.27 118.65) (end 129.625 118.65) (width 0.25) (layer "F.Cu") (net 32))
 (segment (start 140.335 103.505) (end 140.335 104.14) (width 0.25) (layer "F.Cu") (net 32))
 (via (at 140.335 104.14) (size 0.8) (drill 0.4) (layers "F.Cu" "B.Cu") (free) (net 32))
 (via (at 137.16 104.14) (size 0.8) (drill 0.4) (layers "F.Cu" "B.Cu") (free) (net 32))
 (segment (start 137.16 104.14) (end 140.335 104.14) (width 0.25) (layer "B.Cu") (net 32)))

